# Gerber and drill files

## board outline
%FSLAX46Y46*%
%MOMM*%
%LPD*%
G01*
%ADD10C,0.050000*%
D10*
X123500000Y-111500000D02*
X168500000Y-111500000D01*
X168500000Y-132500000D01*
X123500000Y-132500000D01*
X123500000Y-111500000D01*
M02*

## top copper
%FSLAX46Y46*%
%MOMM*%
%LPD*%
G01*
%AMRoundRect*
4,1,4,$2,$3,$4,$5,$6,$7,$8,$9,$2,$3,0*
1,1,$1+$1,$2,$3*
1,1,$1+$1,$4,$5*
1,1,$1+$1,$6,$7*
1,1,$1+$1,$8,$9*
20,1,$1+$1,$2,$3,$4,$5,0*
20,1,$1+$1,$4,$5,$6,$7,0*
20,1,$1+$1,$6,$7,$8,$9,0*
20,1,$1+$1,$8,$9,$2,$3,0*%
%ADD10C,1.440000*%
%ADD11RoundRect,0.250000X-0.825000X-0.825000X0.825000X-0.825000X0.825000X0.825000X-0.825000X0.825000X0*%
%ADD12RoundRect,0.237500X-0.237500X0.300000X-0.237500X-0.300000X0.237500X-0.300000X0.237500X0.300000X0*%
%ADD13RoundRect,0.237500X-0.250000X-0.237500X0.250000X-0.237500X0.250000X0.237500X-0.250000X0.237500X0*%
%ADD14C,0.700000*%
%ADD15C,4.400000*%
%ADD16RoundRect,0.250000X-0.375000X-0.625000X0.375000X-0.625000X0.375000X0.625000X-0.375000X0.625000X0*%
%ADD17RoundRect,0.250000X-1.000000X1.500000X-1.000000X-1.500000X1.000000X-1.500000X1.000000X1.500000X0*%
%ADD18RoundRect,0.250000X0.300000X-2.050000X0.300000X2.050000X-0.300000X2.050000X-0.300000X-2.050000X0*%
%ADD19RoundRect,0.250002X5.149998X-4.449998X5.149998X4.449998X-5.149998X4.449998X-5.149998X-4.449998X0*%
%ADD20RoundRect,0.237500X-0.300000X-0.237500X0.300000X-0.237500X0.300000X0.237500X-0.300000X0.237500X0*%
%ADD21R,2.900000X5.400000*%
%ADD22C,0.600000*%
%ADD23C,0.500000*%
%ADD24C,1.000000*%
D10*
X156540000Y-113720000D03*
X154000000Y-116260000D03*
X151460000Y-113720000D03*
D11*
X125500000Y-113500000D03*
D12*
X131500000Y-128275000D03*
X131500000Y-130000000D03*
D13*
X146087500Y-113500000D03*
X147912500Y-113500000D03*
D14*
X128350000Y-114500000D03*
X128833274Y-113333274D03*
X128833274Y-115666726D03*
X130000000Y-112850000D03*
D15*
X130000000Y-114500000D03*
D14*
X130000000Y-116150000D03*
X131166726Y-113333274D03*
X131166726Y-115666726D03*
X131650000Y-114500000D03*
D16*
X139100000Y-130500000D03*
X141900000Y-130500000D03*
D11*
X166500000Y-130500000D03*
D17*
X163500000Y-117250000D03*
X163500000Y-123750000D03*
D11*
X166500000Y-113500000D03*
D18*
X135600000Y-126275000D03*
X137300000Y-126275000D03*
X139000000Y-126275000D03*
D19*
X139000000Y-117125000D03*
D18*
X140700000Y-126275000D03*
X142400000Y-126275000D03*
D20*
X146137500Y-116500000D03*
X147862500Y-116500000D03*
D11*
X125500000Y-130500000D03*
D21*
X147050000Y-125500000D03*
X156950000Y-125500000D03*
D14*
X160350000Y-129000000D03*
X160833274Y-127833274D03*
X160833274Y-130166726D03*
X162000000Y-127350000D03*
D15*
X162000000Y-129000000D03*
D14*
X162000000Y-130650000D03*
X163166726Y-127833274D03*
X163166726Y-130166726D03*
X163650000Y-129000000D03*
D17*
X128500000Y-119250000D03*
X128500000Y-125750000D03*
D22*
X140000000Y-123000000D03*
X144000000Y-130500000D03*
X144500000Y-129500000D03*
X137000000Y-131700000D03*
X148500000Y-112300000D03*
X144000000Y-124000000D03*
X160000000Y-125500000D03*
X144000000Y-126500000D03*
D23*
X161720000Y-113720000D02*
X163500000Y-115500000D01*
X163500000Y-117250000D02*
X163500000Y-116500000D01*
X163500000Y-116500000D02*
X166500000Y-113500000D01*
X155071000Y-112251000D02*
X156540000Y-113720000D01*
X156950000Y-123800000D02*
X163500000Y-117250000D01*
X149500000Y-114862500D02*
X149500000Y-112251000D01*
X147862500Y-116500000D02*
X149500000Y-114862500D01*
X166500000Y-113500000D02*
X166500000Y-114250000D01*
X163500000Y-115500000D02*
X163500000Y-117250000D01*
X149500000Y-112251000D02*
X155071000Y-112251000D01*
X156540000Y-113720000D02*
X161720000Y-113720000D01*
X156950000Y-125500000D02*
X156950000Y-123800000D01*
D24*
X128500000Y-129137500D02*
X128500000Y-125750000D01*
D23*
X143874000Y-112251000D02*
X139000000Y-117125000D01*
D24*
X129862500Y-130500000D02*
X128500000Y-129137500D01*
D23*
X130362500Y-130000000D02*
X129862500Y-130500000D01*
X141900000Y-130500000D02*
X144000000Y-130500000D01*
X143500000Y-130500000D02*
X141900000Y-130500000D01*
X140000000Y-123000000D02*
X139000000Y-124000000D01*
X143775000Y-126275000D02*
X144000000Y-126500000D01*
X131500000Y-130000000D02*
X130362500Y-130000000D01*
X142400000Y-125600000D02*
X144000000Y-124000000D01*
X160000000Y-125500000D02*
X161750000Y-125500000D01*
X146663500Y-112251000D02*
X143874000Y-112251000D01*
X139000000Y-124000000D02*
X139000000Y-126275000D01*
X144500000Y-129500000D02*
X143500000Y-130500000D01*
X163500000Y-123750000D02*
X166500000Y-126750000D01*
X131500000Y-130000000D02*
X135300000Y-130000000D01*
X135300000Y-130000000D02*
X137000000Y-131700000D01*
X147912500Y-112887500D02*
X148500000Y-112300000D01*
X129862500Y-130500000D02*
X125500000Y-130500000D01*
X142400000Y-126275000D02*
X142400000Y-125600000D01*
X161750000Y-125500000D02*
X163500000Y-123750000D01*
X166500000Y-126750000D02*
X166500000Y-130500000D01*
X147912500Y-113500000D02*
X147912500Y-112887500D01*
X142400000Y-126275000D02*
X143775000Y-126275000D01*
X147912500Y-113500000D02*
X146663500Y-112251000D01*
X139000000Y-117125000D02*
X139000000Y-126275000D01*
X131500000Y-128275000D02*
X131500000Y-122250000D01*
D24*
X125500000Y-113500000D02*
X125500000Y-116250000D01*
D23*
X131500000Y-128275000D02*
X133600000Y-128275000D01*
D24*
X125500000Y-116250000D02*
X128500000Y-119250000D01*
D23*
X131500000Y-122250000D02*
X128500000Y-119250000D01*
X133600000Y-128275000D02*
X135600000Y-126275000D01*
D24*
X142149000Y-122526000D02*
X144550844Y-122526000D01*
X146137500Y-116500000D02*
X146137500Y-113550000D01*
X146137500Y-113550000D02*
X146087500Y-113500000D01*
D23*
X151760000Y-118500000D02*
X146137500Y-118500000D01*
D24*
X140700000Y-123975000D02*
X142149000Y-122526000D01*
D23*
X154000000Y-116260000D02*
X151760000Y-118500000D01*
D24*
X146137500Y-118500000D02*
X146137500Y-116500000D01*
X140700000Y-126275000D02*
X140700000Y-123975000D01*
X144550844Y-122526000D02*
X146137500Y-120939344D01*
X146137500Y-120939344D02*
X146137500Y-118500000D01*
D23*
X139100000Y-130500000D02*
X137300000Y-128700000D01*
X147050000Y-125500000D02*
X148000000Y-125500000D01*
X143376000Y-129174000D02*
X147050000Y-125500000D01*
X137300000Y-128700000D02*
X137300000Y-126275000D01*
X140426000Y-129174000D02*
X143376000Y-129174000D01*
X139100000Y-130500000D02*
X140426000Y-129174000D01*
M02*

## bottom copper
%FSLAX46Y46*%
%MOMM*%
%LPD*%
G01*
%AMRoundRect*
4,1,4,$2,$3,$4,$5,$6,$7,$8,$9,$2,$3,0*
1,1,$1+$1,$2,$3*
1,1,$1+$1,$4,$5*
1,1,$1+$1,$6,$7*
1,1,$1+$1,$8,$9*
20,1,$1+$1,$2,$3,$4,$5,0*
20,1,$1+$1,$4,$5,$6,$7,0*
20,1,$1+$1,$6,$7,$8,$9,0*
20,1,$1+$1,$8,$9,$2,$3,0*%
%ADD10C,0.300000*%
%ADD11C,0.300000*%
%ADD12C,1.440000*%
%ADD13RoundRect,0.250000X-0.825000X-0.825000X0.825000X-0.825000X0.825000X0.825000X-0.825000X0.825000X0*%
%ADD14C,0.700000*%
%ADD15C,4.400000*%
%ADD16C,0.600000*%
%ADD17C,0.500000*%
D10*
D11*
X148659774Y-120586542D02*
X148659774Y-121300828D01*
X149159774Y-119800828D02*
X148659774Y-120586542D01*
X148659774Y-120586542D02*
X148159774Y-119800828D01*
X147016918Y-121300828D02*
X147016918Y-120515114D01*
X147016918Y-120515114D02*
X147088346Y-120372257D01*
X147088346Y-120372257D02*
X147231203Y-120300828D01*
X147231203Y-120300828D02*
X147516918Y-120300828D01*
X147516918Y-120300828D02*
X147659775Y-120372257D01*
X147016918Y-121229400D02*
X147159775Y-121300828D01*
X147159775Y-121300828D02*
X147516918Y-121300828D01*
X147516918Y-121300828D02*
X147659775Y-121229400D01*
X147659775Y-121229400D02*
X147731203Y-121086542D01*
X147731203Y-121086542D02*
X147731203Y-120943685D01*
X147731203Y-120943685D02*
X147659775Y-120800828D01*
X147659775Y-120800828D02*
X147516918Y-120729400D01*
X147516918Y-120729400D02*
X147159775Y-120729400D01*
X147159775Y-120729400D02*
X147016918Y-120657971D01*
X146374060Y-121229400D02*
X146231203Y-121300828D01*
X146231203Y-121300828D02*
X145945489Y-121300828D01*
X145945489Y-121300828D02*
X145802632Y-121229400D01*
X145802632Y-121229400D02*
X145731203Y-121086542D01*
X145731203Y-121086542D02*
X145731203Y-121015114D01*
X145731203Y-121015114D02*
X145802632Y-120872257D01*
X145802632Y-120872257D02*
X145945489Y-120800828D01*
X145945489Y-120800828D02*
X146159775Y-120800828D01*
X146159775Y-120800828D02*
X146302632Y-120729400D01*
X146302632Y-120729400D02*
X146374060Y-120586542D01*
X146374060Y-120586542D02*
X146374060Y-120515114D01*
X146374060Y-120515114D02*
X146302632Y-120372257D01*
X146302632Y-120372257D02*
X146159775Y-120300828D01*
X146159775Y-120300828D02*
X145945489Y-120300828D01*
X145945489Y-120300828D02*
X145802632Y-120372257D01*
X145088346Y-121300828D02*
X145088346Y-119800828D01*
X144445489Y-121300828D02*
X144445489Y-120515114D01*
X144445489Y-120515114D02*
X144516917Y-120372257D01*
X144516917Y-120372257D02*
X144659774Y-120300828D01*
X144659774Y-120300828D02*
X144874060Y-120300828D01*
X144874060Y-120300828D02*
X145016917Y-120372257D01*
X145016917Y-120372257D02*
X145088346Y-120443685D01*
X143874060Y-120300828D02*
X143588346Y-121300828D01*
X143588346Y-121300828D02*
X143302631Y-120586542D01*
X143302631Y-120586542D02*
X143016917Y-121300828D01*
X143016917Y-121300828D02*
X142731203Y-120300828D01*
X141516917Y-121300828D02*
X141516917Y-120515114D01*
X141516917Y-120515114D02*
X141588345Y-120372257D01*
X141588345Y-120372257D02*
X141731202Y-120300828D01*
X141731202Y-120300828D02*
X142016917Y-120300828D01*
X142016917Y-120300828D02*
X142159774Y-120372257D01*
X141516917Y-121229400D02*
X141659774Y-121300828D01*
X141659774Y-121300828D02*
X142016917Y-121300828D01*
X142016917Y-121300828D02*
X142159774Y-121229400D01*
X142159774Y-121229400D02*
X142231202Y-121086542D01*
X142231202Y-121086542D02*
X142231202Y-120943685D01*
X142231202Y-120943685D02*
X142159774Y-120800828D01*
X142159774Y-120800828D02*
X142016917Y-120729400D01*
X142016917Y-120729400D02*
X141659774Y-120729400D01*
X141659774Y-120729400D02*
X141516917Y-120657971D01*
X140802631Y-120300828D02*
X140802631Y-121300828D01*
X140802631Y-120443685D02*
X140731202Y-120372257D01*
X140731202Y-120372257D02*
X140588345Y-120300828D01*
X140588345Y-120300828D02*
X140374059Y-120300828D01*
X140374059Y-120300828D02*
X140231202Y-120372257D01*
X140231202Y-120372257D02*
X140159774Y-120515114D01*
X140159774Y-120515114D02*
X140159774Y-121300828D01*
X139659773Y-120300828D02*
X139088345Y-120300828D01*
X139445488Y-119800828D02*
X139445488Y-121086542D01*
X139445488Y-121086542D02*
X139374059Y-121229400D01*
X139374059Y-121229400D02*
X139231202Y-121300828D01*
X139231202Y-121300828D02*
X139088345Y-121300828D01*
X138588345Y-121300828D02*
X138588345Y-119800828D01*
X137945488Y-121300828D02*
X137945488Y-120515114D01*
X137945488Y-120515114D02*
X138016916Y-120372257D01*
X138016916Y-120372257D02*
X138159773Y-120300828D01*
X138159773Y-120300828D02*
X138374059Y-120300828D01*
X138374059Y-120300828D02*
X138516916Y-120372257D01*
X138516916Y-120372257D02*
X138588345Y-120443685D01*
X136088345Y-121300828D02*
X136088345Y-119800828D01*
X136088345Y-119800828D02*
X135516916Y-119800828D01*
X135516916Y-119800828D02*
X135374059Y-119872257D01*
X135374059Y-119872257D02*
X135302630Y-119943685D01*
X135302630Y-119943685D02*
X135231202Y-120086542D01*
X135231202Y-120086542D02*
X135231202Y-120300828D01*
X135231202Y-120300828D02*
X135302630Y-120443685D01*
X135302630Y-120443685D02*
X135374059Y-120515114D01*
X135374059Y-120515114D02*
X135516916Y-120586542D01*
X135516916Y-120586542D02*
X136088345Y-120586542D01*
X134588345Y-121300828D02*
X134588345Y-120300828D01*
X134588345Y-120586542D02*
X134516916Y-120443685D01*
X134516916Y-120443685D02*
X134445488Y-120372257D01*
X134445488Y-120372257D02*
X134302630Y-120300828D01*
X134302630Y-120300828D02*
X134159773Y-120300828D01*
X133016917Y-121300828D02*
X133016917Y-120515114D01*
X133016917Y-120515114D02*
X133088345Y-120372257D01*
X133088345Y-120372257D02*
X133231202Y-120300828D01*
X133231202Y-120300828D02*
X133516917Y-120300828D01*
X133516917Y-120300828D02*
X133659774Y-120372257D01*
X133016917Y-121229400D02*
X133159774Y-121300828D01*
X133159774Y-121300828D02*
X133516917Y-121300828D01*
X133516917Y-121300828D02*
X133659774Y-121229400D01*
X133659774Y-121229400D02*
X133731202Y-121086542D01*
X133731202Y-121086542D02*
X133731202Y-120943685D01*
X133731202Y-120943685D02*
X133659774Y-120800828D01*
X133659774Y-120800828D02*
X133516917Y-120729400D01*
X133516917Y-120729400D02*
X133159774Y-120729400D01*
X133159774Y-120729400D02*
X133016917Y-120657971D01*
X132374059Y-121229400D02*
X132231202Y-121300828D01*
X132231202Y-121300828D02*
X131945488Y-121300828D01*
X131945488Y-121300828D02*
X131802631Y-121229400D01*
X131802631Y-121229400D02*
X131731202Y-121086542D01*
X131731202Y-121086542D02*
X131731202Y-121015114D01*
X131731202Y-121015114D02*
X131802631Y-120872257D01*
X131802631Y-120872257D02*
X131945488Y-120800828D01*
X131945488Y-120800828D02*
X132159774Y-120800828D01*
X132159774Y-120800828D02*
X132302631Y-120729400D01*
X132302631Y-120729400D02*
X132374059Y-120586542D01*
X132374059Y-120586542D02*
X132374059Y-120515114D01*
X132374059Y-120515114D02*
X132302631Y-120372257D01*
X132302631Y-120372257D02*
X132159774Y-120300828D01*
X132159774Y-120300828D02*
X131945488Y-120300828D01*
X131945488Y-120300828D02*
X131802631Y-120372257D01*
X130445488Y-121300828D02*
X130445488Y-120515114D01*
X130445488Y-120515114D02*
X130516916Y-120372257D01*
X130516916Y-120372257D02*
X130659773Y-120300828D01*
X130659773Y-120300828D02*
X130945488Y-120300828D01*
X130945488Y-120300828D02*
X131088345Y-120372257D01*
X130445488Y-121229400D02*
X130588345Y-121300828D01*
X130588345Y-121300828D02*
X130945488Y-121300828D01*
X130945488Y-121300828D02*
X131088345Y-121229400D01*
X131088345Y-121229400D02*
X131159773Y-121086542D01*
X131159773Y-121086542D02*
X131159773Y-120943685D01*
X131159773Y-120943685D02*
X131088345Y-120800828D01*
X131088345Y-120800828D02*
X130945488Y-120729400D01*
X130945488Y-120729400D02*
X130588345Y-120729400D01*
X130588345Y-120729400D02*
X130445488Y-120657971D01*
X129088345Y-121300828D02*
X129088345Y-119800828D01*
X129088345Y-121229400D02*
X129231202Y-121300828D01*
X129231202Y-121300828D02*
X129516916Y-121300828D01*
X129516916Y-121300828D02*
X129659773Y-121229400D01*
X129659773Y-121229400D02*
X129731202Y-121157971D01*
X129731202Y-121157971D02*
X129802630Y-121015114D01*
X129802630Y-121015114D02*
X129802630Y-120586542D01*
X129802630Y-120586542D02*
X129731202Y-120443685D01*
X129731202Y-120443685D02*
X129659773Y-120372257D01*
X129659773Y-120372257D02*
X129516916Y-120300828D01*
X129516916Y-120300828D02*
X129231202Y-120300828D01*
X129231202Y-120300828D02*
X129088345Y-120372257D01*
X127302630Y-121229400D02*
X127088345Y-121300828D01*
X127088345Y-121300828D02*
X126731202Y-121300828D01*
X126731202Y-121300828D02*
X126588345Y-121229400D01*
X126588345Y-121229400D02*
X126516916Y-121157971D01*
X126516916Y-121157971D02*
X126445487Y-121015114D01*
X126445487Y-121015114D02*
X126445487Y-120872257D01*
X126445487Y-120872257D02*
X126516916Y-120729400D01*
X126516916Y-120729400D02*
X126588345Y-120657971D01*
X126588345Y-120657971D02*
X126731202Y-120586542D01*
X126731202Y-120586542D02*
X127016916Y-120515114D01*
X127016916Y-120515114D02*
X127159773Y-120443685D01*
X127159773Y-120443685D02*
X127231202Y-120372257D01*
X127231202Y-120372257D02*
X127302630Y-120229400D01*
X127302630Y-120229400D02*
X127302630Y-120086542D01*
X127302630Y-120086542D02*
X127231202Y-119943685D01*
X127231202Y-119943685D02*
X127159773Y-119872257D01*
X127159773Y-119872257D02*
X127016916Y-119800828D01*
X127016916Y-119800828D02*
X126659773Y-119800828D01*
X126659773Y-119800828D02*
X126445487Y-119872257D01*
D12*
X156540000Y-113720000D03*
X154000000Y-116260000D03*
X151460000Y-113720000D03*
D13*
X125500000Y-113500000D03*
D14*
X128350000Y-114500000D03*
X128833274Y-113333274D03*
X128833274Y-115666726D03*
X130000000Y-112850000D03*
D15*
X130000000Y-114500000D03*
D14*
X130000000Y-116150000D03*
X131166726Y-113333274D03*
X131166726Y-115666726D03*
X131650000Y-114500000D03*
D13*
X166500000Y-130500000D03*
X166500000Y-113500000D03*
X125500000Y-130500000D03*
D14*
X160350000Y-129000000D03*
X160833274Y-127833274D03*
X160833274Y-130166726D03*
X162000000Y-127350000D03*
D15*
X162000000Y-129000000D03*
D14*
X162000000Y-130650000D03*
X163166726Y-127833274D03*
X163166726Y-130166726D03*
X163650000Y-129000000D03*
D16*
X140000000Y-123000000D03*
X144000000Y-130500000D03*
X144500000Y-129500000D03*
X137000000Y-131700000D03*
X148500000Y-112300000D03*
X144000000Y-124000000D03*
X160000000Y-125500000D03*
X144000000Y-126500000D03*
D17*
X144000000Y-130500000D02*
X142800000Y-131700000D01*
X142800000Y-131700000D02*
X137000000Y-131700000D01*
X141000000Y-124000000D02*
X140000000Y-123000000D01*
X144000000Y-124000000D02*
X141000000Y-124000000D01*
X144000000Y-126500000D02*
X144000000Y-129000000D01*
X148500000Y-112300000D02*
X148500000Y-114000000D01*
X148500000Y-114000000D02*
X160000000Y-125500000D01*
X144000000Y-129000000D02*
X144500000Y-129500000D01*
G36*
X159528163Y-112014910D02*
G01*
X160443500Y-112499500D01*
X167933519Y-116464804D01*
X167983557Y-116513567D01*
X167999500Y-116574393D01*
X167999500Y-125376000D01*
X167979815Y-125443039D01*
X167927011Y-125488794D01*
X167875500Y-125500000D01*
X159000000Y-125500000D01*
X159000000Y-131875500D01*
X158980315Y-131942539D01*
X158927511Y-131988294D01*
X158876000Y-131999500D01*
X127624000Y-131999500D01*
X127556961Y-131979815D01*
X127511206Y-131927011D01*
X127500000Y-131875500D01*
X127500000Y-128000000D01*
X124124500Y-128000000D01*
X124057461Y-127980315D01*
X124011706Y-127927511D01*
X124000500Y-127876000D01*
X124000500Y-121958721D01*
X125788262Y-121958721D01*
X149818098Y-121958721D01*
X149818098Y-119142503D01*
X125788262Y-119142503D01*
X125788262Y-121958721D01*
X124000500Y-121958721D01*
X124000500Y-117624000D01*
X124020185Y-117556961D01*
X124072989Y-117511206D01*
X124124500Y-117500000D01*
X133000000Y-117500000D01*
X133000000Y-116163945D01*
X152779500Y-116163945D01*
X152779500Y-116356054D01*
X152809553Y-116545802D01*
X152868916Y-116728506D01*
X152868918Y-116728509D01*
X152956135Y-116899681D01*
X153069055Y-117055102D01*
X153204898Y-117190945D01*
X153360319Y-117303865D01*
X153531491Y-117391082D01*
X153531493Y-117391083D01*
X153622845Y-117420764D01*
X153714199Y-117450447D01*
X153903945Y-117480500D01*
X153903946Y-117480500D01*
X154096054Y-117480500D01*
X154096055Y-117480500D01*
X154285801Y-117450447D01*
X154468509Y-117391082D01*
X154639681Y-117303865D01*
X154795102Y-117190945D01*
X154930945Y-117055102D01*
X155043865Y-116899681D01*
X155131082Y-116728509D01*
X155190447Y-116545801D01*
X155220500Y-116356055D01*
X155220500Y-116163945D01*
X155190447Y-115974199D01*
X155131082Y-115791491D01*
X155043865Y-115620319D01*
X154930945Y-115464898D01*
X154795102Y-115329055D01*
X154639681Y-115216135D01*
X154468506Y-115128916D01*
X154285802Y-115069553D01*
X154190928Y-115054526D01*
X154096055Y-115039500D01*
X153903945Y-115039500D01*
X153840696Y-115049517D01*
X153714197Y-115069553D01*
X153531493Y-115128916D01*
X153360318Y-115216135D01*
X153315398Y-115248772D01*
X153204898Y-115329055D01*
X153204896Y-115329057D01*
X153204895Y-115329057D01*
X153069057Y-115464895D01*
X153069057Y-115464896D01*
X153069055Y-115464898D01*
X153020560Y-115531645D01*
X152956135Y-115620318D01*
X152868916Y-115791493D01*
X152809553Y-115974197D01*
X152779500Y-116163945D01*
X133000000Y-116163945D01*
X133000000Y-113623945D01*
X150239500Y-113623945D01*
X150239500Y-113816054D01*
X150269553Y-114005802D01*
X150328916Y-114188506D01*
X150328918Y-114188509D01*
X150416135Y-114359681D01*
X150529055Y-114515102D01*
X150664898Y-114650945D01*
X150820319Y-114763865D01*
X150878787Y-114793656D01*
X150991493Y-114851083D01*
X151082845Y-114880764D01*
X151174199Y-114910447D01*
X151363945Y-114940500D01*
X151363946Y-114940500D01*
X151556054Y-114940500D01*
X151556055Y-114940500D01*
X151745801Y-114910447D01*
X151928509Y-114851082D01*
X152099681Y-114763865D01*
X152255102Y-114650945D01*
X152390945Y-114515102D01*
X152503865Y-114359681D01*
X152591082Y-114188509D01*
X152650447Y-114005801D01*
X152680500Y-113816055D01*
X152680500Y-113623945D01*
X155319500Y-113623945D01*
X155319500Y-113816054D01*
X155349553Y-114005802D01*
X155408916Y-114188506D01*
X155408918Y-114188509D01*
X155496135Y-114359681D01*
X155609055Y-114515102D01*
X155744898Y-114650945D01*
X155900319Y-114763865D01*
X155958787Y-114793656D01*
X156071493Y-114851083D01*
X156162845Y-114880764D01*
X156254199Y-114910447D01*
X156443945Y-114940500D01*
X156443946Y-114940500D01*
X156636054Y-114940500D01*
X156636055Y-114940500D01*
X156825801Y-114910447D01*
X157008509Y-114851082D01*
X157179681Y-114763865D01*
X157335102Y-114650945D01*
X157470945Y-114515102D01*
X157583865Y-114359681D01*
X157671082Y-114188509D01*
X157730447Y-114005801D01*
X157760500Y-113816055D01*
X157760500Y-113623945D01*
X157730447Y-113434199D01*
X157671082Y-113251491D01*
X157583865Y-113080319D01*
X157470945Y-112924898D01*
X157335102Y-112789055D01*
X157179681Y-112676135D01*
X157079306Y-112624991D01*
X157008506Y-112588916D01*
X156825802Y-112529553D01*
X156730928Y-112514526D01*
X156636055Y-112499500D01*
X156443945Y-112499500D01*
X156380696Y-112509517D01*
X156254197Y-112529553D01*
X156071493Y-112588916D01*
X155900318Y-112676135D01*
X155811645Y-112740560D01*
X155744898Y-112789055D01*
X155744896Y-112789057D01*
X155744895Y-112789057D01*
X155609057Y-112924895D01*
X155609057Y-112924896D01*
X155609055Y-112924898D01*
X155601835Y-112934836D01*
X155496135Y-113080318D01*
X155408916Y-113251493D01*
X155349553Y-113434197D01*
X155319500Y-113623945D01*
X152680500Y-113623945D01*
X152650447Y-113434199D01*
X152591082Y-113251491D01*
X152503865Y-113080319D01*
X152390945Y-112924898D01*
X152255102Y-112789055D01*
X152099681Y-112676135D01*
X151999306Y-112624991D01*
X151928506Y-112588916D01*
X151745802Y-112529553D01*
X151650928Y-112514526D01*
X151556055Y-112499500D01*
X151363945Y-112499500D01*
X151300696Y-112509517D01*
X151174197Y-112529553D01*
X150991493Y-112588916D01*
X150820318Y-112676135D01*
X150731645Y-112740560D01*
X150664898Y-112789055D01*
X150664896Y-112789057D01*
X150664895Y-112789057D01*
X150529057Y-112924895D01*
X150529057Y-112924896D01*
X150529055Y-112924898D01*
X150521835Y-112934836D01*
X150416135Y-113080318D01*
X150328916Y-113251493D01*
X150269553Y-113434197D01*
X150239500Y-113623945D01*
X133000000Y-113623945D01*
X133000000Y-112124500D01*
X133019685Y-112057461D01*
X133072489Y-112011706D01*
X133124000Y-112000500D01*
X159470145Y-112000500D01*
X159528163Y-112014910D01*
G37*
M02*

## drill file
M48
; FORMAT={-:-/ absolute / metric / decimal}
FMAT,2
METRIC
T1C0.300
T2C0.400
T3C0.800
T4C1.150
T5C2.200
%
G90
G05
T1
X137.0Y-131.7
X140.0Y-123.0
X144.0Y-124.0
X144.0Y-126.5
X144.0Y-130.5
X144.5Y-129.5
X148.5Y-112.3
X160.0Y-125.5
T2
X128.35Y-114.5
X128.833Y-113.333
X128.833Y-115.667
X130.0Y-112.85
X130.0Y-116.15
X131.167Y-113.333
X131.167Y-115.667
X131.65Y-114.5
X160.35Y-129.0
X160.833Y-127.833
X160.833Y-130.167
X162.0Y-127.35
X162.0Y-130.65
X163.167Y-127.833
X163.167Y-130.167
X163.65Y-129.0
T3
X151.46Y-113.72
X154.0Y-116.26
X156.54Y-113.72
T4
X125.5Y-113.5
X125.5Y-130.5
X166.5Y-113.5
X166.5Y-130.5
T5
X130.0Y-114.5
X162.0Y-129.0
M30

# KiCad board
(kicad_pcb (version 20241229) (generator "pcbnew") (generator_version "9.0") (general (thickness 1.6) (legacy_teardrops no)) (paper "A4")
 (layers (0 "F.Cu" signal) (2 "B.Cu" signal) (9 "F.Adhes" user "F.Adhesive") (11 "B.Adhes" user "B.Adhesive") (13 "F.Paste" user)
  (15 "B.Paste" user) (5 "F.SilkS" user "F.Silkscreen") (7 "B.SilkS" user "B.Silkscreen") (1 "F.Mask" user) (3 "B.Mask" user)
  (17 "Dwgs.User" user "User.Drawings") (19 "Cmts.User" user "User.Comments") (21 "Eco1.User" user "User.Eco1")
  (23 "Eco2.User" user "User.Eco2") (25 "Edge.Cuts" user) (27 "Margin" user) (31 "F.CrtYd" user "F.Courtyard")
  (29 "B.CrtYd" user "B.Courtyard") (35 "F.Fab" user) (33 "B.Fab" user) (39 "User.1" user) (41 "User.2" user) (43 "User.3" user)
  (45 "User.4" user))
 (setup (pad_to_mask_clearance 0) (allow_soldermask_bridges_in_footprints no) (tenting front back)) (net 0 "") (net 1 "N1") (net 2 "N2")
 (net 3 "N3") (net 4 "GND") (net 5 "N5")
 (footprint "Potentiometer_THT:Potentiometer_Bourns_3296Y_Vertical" (layer "F.Cu") (at 156.54 113.72)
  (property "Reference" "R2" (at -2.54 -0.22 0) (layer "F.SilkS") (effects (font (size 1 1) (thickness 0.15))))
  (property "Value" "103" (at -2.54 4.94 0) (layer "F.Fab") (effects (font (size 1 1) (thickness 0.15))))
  (pad "1" thru_hole circle (at 0 0) (size 1.44 1.44) (drill 0.8) (layers "*.Cu" "*.Mask") (remove_unused_layers no) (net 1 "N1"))
  (pad "2" thru_hole circle (at -2.54 2.54) (size 1.44 1.44) (drill 0.8) (layers "*.Cu" "*.Mask") (remove_unused_layers no) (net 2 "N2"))
  (pad "3" thru_hole circle (at -5.08 0) (size 1.44 1.44) (drill 0.8) (layers "*.Cu" "*.Mask") (remove_unused_layers no)))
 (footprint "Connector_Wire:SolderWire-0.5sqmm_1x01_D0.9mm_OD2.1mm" (layer "F.Cu") (at 125.5 113.5)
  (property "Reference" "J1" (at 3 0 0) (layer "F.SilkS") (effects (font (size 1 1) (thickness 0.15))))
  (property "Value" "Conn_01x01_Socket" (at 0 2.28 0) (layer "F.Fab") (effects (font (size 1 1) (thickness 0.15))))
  (pad "1" thru_hole roundrect (at 0 0) (size 2.15 2.15) (drill 1.15) (layers "*.Cu" "*.Mask") (remove_unused_layers no)
   (roundrect_rratio 0.116279) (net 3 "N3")))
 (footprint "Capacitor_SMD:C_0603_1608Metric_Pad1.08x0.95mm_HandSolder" (layer "F.Cu") (at 131.5 129.1375 -90)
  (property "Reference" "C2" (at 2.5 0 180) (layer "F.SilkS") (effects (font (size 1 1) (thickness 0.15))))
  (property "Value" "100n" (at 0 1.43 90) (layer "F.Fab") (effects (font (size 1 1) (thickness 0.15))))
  (pad "1" smd roundrect (at -0.8625 0 270) (size 1.075 0.95) (layers "F.Cu" "F.Mask" "F.Paste") (roundrect_rratio 0.25) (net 3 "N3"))
  (pad "2" smd roundrect (at 0.8625 0 270) (size 1.075 0.95) (layers "F.Cu" "F.Mask" "F.Paste") (roundrect_rratio 0.25) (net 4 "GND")))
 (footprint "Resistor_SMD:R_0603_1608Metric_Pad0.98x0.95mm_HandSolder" (layer "F.Cu") (at 147 113.5)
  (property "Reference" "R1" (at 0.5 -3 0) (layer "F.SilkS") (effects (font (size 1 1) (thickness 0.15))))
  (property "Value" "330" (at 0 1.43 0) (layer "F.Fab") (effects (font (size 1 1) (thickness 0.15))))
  (pad "1" smd roundrect (at -0.9125 0) (size 0.975 0.95) (layers "F.Cu" "F.Mask" "F.Paste") (roundrect_rratio 0.25) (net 2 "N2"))
  (pad "2" smd roundrect (at 0.9125 0) (size 0.975 0.95) (layers "F.Cu" "F.Mask" "F.Paste") (roundrect_rratio 0.25) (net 4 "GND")))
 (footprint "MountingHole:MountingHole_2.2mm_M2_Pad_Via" (layer "F.Cu") (at 130 114.5)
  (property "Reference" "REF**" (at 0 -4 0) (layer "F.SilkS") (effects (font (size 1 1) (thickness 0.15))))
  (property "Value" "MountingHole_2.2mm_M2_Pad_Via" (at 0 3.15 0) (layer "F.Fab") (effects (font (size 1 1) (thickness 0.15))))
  (pad "1" thru_hole circle (at -1.65 0) (size 0.7 0.7) (drill 0.4) (layers "*.Cu" "*.Mask") (remove_unused_layers no) (zone_connect 2))
  (pad "1" thru_hole circle (at -1.166726 -1.166726) (size 0.7 0.7) (drill 0.4) (layers "*.Cu" "*.Mask") (remove_unused_layers no)
   (zone_connect 2))
  (pad "1" thru_hole circle (at -1.166726 1.166726) (size 0.7 0.7) (drill 0.4) (layers "*.Cu" "*.Mask") (remove_unused_layers no)
   (zone_connect 2))
  (pad "1" thru_hole circle (at 0 -1.65) (size 0.7 0.7) (drill 0.4) (layers "*.Cu" "*.Mask") (remove_unused_layers no) (zone_connect 2))
  (pad "1" thru_hole circle (at 0 0) (size 4.4 4.4) (drill 2.2) (layers "*.Cu" "*.Mask") (remove_unused_layers no) (zone_connect 2))
  (pad "1" thru_hole circle (at 0 1.65) (size 0.7 0.7) (drill 0.4) (layers "*.Cu" "*.Mask") (remove_unused_layers no) (zone_connect 2))
  (pad "1" thru_hole circle (at 1.166726 -1.166726) (size 0.7 0.7) (drill 0.4) (layers "*.Cu" "*.Mask") (remove_unused_layers no)
   (zone_connect 2))
  (pad "1" thru_hole circle (at 1.166726 1.166726) (size 0.7 0.7) (drill 0.4) (layers "*.Cu" "*.Mask") (remove_unused_layers no)
   (zone_connect 2))
  (pad "1" thru_hole circle (at 1.65 0) (size 0.7 0.7) (drill 0.4) (layers "*.Cu" "*.Mask") (remove_unused_layers no) (zone_connect 2)))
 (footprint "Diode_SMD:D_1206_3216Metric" (layer "F.Cu") (at 140.5 130.5)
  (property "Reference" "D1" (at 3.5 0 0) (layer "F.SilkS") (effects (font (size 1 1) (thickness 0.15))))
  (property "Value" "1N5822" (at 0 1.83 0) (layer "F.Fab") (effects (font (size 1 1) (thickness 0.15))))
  (pad "1" smd roundrect (at -1.4 0) (size 1.25 1.75) (layers "F.Cu" "F.Mask" "F.Paste") (roundrect_rratio 0.2) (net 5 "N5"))
  (pad "2" smd roundrect (at 1.4 0) (size 1.25 1.75) (layers "F.Cu" "F.Mask" "F.Paste") (roundrect_rratio 0.2) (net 4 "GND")))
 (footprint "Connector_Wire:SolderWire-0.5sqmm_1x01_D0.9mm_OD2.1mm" (layer "F.Cu") (at 166.5 130.5)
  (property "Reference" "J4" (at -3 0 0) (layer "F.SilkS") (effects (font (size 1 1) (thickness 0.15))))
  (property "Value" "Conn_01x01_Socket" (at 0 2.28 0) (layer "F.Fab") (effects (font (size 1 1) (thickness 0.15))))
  (pad "1" thru_hole roundrect (at 0 0) (size 2.15 2.15) (drill 1.15) (layers "*.Cu" "*.Mask") (remove_unused_layers no)
   (roundrect_rratio 0.116279) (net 4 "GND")))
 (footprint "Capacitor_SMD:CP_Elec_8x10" (layer "F.Cu") (at 163.5 120.5 -90)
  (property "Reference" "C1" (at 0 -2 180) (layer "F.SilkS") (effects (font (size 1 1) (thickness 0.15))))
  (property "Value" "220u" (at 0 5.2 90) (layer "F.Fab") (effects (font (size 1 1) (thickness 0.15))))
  (pad "1" smd roundrect (at -3.25 0 270) (size 3.5 2.5) (layers "F.Cu" "F.Mask" "F.Paste") (roundrect_rratio 0.1) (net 1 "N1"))
  (pad "2" smd roundrect (at 3.25 0 270) (size 3.5 2.5) (layers "F.Cu" "F.Mask" "F.Paste") (roundrect_rratio 0.1) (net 4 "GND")))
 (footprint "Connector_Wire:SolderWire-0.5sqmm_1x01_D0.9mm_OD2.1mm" (layer "F.Cu") (at 166.5 113.5)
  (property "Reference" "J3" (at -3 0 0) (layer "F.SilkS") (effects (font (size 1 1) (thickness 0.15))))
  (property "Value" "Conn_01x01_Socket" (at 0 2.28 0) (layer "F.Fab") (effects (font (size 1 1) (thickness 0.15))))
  (pad "1" thru_hole roundrect (at 0 0) (size 2.15 2.15) (drill 1.15) (layers "*.Cu" "*.Mask") (remove_unused_layers no)
   (roundrect_rratio 0.116279) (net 1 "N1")))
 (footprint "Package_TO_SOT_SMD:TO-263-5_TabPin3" (layer "F.Cu") (at 139 118.625 90)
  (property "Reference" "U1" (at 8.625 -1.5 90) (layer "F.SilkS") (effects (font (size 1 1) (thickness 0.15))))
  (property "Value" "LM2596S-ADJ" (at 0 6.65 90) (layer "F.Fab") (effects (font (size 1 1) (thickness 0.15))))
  (pad "" smd roundrect (at -0.925 -2.775 90) (size 4.55 5.25) (layers "F.Paste") (roundrect_rratio 0.054945))
  (pad "" smd roundrect (at -0.925 2.775 90) (size 4.55 5.25) (layers "F.Paste") (roundrect_rratio 0.054945))
  (pad "" smd roundrect (at 3.925 -2.775 90) (size 4.55 5.25) (layers "F.Paste") (roundrect_rratio 0.054945))
  (pad "" smd roundrect (at 3.925 2.775 90) (size 4.55 5.25) (layers "F.Paste") (roundrect_rratio 0.054945))
  (pad "1" smd roundrect (at -7.65 -3.4 90) (size 4.6 1.1) (layers "F.Cu" "F.Mask" "F.Paste") (roundrect_rratio 0.227273) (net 3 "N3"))
  (pad "2" smd roundrect (at -7.65 -1.7 90) (size 4.6 1.1) (layers "F.Cu" "F.Mask" "F.Paste") (roundrect_rratio 0.227273) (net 5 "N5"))
  (pad "3" smd roundrect (at -7.65 0 90) (size 4.6 1.1) (layers "F.Cu" "F.Mask" "F.Paste") (roundrect_rratio 0.227273) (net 4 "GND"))
  (pad "3" smd roundrect (at 1.5 0 90) (size 9.4 10.8) (layers "F.Cu" "F.Mask") (roundrect_rratio 0.026596) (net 4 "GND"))
  (pad "4" smd roundrect (at -7.65 1.7 90) (size 4.6 1.1) (layers "F.Cu" "F.Mask" "F.Paste") (roundrect_rratio 0.227273) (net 2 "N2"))
  (pad "5" smd roundrect (at -7.65 3.4 90) (size 4.6 1.1) (layers "F.Cu" "F.Mask" "F.Paste") (roundrect_rratio 0.227273) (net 4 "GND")))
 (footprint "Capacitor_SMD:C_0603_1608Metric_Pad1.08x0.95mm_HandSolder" (layer "F.Cu") (at 147 116.5)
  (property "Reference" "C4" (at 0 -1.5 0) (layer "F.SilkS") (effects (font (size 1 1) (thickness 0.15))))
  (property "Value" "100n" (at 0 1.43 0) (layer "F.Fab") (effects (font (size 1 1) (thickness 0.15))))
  (pad "1" smd roundrect (at -0.8625 0) (size 1.075 0.95) (layers "F.Cu" "F.Mask" "F.Paste") (roundrect_rratio 0.25) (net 2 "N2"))
  (pad "2" smd roundrect (at 0.8625 0) (size 1.075 0.95) (layers "F.Cu" "F.Mask" "F.Paste") (roundrect_rratio 0.25) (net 1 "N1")))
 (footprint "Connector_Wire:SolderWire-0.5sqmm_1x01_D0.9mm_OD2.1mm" (layer "F.Cu") (at 125.5 130.5)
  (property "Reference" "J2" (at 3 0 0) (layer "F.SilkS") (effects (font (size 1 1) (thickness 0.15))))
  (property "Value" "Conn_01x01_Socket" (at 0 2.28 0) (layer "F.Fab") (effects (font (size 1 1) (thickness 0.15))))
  (pad "1" thru_hole roundrect (at 0 0) (size 2.15 2.15) (drill 1.15) (layers "*.Cu" "*.Mask") (remove_unused_layers no)
   (roundrect_rratio 0.116279) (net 4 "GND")))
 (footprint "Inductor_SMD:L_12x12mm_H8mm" (layer "F.Cu") (at 152 125.5)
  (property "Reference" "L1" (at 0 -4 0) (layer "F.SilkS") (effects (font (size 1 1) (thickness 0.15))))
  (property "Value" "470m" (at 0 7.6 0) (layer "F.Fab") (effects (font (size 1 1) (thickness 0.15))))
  (pad "1" smd rect (at -4.95 0) (size 2.9 5.4) (layers "F.Cu" "F.Mask" "F.Paste") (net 5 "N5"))
  (pad "2" smd rect (at 4.95 0) (size 2.9 5.4) (layers "F.Cu" "F.Mask" "F.Paste") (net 1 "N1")))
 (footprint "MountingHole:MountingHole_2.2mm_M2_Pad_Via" (layer "F.Cu") (at 162 129)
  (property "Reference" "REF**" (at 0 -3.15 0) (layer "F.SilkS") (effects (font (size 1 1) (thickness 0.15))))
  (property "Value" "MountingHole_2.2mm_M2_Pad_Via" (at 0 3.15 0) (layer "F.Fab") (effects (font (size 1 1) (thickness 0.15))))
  (pad "1" thru_hole circle (at -1.65 0) (size 0.7 0.7) (drill 0.4) (layers "*.Cu" "*.Mask") (remove_unused_layers no) (zone_connect 2))
  (pad "1" thru_hole circle (at -1.166726 -1.166726) (size 0.7 0.7) (drill 0.4) (layers "*.Cu" "*.Mask") (remove_unused_layers no)
   (zone_connect 2))
  (pad "1" thru_hole circle (at -1.166726 1.166726) (size 0.7 0.7) (drill 0.4) (layers "*.Cu" "*.Mask") (remove_unused_layers no)
   (zone_connect 2))
  (pad "1" thru_hole circle (at 0 -1.65) (size 0.7 0.7) (drill 0.4) (layers "*.Cu" "*.Mask") (remove_unused_layers no) (zone_connect 2))
  (pad "1" thru_hole circle (at 0 0) (size 4.4 4.4) (drill 2.2) (layers "*.Cu" "*.Mask") (remove_unused_layers no) (zone_connect 2))
  (pad "1" thru_hole circle (at 0 1.65) (size 0.7 0.7) (drill 0.4) (layers "*.Cu" "*.Mask") (remove_unused_layers no) (zone_connect 2))
  (pad "1" thru_hole circle (at 1.166726 -1.166726) (size 0.7 0.7) (drill 0.4) (layers "*.Cu" "*.Mask") (remove_unused_layers no)
   (zone_connect 2))
  (pad "1" thru_hole circle (at 1.166726 1.166726) (size 0.7 0.7) (drill 0.4) (layers "*.Cu" "*.Mask") (remove_unused_layers no)
   (zone_connect 2))
  (pad "1" thru_hole circle (at 1.65 0) (size 0.7 0.7) (drill 0.4) (layers "*.Cu" "*.Mask") (remove_unused_layers no) (zone_connect 2)))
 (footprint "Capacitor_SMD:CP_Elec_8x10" (layer "F.Cu") (at 128.5 122.5 -90)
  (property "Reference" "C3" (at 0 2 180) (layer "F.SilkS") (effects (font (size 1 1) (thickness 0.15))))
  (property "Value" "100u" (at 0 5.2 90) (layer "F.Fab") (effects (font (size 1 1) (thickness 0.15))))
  (pad "1" smd roundrect (at -3.25 0 270) (size 3.5 2.5) (layers "F.Cu" "F.Mask" "F.Paste") (roundrect_rratio 0.1) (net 3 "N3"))
  (pad "2" smd roundrect (at 3.25 0 270) (size 3.5 2.5) (layers "F.Cu" "F.Mask" "F.Paste") (roundrect_rratio 0.1) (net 4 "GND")))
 (gr_rect (start 123.5 111.5) (end 168.5 132.5) (stroke (width 0.05) (type default)) (fill no) (layer "Edge.Cuts"))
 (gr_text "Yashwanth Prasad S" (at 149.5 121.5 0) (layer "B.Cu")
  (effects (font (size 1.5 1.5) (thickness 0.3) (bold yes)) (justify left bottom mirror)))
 (segment (start 161.72 113.72) (end 163.5 115.5) (width 0.5) (layer "F.Cu") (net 1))
 (segment (start 163.5 117.25) (end 163.5 116.5) (width 0.5) (layer "F.Cu") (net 1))
 (segment (start 163.5 116.5) (end 166.5 113.5) (width 0.5) (layer "F.Cu") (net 1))
 (segment (start 155.071 112.251) (end 156.54 113.72) (width 0.5) (layer "F.Cu") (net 1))
 (segment (start 156.95 123.8) (end 163.5 117.25) (width 0.5) (layer "F.Cu") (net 1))
 (segment (start 149.5 114.8625) (end 149.5 112.251) (width 0.5) (layer "F.Cu") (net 1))
 (segment (start 147.8625 116.5) (end 149.5 114.8625) (width 0.5) (layer "F.Cu") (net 1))
 (segment (start 166.5 113.5) (end 166.5 114.25) (width 0.5) (layer "F.Cu") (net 1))
 (segment (start 163.5 115.5) (end 163.5 117.25) (width 0.5) (layer "F.Cu") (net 1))
 (segment (start 149.5 112.251) (end 155.071 112.251) (width 0.5) (layer "F.Cu") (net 1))
 (segment (start 156.54 113.72) (end 161.72 113.72) (width 0.5) (layer "F.Cu") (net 1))
 (segment (start 156.95 125.5) (end 156.95 123.8) (width 0.5) (layer "F.Cu") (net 1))
 (segment (start 128.5 129.1375) (end 128.5 125.75) (width 1) (layer "F.Cu") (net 4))
 (segment (start 143.874 112.251) (end 139 117.125) (width 0.5) (layer "F.Cu") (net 4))
 (segment (start 129.8625 130.5) (end 128.5 129.1375) (width 1) (layer "F.Cu") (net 4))
 (segment (start 130.3625 130) (end 129.8625 130.5) (width 0.5) (layer "F.Cu") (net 4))
 (segment (start 141.9 130.5) (end 144 130.5) (width 0.5) (layer "F.Cu") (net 4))
 (segment (start 143.5 130.5) (end 141.9 130.5) (width 0.5) (layer "F.Cu") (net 4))
 (segment (start 140 123) (end 139 124) (width 0.5) (layer "F.Cu") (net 4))
 (segment (start 143.775 126.275) (end 144 126.5) (width 0.5) (layer "F.Cu") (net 4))
 (segment (start 131.5 130) (end 130.3625 130) (width 0.5) (layer "F.Cu") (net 4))
 (segment (start 142.4 125.6) (end 144 124) (width 0.5) (layer "F.Cu") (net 4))
 (segment (start 160 125.5) (end 161.75 125.5) (width 0.5) (layer "F.Cu") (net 4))
 (segment (start 146.6635 112.251) (end 143.874 112.251) (width 0.5) (layer "F.Cu") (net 4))
 (segment (start 139 124) (end 139 126.275) (width 0.5) (layer "F.Cu") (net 4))
 (segment (start 144.5 129.5) (end 143.5 130.5) (width 0.5) (layer "F.Cu") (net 4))
 (segment (start 163.5 123.75) (end 166.5 126.75) (width 0.5) (layer "F.Cu") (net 4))
 (segment (start 131.5 130) (end 135.3 130) (width 0.5) (layer "F.Cu") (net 4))
 (segment (start 135.3 130) (end 137 131.7) (width 0.5) (layer "F.Cu") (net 4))
 (segment (start 147.9125 112.8875) (end 148.5 112.3) (width 0.5) (layer "F.Cu") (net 4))
 (segment (start 129.8625 130.5) (end 125.5 130.5) (width 0.5) (layer "F.Cu") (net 4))
 (segment (start 142.4 126.275) (end 142.4 125.6) (width 0.5) (layer "F.Cu") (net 4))
 (segment (start 161.75 125.5) (end 163.5 123.75) (width 0.5) (layer "F.Cu") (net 4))
 (segment (start 166.5 126.75) (end 166.5 130.5) (width 0.5) (layer "F.Cu") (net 4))
 (segment (start 147.9125 113.5) (end 147.9125 112.8875) (width 0.5) (layer "F.Cu") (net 4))
 (segment (start 142.4 126.275) (end 143.775 126.275) (width 0.5) (layer "F.Cu") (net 4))
 (segment (start 147.9125 113.5) (end 146.6635 112.251) (width 0.5) (layer "F.Cu") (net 4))
 (segment (start 139 117.125) (end 139 126.275) (width 0.5) (layer "F.Cu") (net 4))
 (via (at 140 123) (size 0.6) (drill 0.3) (layers "F.Cu" "B.Cu") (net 4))
 (via (at 144 130.5) (size 0.6) (drill 0.3) (layers "F.Cu" "B.Cu") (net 4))
 (via (at 144.5 129.5) (size 0.6) (drill 0.3) (layers "F.Cu" "B.Cu") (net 4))
 (via (at 137 131.7) (size 0.6) (drill 0.3) (layers "F.Cu" "B.Cu") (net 4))
 (via (at 148.5 112.3) (size 0.6) (drill 0.3) (layers "F.Cu" "B.Cu") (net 4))
 (via (at 144 124) (size 0.6) (drill 0.3) (layers "F.Cu" "B.Cu") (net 4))
 (via (at 160 125.5) (size 0.6) (drill 0.3) (layers "F.Cu" "B.Cu") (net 4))
 (via (at 144 126.5) (size 0.6) (drill 0.3) (layers "F.Cu" "B.Cu") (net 4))
 (segment (start 144 130.5) (end 142.8 131.7) (width 0.5) (layer "B.Cu") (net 4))
 (segment (start 142.8 131.7) (end 137 131.7) (width 0.5) (layer "B.Cu") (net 4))
 (segment (start 141 124) (end 140 123) (width 0.5) (layer "B.Cu") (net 4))
 (segment (start 144 124) (end 141 124) (width 0.5) (layer "B.Cu") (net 4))
 (segment (start 144 126.5) (end 144 129) (width 0.5) (layer "B.Cu") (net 4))
 (segment (start 148.5 112.3) (end 148.5 114) (width 0.5) (layer "B.Cu") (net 4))
 (segment (start 148.5 114) (end 160 125.5) (width 0.5) (layer "B.Cu") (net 4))
 (segment (start 144 129) (end 144.5 129.5) (width 0.5) (layer "B.Cu") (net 4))
 (segment (start 131.5 128.275) (end 131.5 122.25) (width 0.5) (layer "F.Cu") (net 3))
 (segment (start 125.5 113.5) (end 125.5 116.25) (width 1) (layer "F.Cu") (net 3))
 (segment (start 131.5 128.275) (end 133.6 128.275) (width 0.5) (layer "F.Cu") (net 3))
 (segment (start 125.5 116.25) (end 128.5 119.25) (width 1) (layer "F.Cu") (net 3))
 (segment (start 131.5 122.25) (end 128.5 119.25) (width 0.5) (layer "F.Cu") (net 3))
 (segment (start 133.6 128.275) (end 135.6 126.275) (width 0.5) (layer "F.Cu") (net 3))
 (segment (start 142.149 122.526) (end 144.550844 122.526) (width 1) (layer "F.Cu") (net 2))
 (segment (start 146.1375 116.5) (end 146.1375 113.55) (width 1) (layer "F.Cu") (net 2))
 (segment (start 146.1375 113.55) (end 146.0875 113.5) (width 1) (layer "F.Cu") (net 2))
 (segment (start 151.76 118.5) (end 146.1375 118.5) (width 0.5) (layer "F.Cu") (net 2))
 (segment (start 140.7 123.975) (end 142.149 122.526) (width 1) (layer "F.Cu") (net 2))
 (segment (start 154 116.26) (end 151.76 118.5) (width 0.5) (layer "F.Cu") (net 2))
 (segment (start 146.1375 118.5) (end 146.1375 116.5) (width 1) (layer "F.Cu") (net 2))
 (segment (start 140.7 126.275) (end 140.7 123.975) (width 1) (layer "F.Cu") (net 2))
 (segment (start 144.550844 122.526) (end 146.1375 120.939344) (width 1) (layer "F.Cu") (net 2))
 (segment (start 146.1375 120.939344) (end 146.1375 118.5) (width 1) (layer "F.Cu") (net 2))
 (segment (start 139.1 130.5) (end 137.3 128.7) (width 0.5) (layer "F.Cu") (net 5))
 (segment (start 147.05 125.5) (end 148 125.5) (width 0.5) (layer "F.Cu") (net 5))
 (segment (start 143.376 129.174) (end 147.05 125.5) (width 0.5) (layer "F.Cu") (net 5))
 (segment (start 137.3 128.7) (end 137.3 126.275) (width 0.5) (layer "F.Cu") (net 5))
 (segment (start 140.426 129.174) (end 143.376 129.174) (width 0.5) (layer "F.Cu") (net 5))
 (segment (start 139.1 130.5) (end 140.426 129.174) (width 0.5) (layer "F.Cu") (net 5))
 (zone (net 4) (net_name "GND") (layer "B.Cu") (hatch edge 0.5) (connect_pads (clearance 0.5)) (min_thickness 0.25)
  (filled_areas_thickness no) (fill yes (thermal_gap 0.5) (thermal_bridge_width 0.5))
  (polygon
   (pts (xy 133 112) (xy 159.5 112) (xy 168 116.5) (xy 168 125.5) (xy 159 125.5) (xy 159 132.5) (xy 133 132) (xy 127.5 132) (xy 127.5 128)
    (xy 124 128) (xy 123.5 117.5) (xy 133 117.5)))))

